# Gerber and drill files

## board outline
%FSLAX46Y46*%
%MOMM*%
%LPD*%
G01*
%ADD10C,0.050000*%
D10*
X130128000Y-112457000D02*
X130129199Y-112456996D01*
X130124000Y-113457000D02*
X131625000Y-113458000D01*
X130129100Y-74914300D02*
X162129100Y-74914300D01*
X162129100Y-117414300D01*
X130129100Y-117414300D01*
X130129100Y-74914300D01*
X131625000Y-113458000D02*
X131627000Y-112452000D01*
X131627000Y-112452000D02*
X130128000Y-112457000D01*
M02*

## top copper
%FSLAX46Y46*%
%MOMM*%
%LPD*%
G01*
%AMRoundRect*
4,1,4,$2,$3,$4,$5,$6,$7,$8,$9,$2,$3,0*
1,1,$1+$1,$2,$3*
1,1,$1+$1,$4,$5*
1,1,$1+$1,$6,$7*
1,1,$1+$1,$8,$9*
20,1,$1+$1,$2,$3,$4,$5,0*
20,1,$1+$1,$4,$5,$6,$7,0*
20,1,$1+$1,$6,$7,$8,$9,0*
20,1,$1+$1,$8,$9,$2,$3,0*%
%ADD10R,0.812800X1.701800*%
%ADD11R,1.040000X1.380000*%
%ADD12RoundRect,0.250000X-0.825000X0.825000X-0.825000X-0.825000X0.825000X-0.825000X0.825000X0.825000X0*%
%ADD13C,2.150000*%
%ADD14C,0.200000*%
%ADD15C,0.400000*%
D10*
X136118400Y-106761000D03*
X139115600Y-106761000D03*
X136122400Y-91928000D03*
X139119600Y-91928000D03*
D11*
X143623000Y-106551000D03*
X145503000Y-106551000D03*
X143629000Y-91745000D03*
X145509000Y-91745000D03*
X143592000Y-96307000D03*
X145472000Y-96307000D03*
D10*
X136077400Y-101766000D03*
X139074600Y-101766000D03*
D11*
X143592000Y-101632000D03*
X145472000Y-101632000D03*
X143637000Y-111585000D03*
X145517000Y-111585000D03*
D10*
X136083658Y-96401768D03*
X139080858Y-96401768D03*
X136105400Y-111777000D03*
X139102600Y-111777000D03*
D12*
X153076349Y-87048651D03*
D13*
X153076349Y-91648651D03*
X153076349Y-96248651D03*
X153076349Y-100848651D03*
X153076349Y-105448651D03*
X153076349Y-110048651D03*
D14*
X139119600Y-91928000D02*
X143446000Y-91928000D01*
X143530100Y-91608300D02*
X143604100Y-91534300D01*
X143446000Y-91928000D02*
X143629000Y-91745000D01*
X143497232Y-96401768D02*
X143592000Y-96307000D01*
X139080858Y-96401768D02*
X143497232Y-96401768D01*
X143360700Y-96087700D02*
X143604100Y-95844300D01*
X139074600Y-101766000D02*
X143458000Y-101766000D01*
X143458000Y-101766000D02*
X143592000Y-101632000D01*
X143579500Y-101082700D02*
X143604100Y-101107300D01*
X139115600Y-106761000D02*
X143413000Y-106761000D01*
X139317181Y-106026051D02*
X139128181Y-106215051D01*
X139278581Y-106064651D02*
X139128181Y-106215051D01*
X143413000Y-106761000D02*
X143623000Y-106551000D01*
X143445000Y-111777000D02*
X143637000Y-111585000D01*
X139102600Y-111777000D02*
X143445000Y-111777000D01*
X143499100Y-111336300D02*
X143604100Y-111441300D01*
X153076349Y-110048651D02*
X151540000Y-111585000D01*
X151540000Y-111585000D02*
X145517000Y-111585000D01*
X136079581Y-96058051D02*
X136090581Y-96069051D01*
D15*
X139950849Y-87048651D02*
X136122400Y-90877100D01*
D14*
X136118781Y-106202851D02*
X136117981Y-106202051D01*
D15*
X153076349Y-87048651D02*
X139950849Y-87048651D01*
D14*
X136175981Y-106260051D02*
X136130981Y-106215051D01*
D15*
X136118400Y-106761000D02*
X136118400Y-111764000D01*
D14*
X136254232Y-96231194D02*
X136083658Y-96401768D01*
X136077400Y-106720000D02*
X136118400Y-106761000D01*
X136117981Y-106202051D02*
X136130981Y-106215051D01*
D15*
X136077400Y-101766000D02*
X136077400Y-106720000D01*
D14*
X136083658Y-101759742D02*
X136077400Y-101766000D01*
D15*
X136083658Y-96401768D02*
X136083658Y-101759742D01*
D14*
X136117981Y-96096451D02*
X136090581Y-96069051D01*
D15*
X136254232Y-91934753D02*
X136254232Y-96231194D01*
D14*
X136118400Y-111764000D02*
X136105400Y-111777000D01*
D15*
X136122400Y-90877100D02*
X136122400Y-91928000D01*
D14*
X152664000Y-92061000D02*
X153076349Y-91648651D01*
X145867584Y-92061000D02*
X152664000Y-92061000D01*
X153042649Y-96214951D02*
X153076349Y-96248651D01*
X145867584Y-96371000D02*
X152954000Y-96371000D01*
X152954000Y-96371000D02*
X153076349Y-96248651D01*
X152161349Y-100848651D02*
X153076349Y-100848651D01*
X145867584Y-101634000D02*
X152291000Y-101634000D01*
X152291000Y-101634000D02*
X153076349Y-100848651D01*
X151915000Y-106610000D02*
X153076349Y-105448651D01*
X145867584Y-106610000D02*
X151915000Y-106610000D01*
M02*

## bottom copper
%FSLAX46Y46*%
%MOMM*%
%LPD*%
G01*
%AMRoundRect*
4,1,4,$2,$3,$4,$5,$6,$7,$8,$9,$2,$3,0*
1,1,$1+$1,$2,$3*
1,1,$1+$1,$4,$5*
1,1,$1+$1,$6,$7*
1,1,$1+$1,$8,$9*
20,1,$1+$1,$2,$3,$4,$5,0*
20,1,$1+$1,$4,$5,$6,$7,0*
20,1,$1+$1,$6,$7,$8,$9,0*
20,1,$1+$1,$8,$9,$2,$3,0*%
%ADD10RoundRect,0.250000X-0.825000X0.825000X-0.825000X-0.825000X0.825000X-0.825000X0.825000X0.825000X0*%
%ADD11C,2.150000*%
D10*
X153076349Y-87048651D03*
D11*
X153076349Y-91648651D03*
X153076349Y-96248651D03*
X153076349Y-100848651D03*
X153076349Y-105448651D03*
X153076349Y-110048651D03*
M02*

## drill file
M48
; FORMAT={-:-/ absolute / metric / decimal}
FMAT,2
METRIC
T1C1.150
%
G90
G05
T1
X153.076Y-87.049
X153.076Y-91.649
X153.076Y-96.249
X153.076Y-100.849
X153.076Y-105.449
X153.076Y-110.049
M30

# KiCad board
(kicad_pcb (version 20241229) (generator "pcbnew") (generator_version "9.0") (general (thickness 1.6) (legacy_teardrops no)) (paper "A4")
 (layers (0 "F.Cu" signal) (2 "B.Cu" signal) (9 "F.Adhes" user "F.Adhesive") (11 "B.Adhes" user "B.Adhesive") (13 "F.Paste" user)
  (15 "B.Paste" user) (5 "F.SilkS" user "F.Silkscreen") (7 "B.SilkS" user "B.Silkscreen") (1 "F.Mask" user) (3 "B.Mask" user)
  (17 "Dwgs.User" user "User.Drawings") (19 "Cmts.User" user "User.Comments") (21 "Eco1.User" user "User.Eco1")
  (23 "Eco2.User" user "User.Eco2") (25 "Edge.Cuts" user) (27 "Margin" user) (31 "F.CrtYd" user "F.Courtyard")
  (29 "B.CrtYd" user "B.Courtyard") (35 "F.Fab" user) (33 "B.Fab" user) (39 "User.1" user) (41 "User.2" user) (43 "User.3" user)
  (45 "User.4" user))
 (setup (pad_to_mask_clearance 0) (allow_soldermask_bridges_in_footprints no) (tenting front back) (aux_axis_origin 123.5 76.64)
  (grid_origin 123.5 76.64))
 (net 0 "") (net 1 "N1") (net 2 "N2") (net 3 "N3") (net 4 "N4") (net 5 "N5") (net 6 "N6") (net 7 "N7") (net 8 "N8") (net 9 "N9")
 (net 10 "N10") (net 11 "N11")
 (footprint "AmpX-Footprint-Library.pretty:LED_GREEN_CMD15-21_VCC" (layer "F.Cu") (at 137.617 106.761)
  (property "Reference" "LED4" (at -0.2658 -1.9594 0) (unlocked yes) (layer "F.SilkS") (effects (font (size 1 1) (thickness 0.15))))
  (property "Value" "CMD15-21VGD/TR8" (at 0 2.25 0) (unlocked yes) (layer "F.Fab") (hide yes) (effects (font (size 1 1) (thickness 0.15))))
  (pad "1" smd rect (at -1.4986 0) (size 0.8128 1.7018) (layers "F.Cu" "F.Mask" "F.Paste") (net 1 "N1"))
  (pad "2" smd rect (at 1.4986 0) (size 0.8128 1.7018) (layers "F.Cu" "F.Mask" "F.Paste") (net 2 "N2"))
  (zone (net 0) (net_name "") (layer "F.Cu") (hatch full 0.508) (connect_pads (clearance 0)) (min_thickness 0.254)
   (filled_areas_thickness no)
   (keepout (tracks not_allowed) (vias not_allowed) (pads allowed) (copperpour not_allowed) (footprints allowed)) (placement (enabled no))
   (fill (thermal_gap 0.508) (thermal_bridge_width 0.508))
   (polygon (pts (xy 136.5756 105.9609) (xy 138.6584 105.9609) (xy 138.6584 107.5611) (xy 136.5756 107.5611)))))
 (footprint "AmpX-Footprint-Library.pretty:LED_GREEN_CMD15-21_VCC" (layer "F.Cu") (at 137.621 91.928)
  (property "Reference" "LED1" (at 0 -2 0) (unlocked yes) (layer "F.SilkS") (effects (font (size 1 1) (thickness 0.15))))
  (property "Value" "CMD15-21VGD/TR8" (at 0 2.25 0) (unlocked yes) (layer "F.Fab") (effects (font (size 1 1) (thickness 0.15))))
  (pad "1" smd rect (at -1.4986 0) (size 0.8128 1.7018) (layers "F.Cu" "F.Mask" "F.Paste") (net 1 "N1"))
  (pad "2" smd rect (at 1.4986 0) (size 0.8128 1.7018) (layers "F.Cu" "F.Mask" "F.Paste") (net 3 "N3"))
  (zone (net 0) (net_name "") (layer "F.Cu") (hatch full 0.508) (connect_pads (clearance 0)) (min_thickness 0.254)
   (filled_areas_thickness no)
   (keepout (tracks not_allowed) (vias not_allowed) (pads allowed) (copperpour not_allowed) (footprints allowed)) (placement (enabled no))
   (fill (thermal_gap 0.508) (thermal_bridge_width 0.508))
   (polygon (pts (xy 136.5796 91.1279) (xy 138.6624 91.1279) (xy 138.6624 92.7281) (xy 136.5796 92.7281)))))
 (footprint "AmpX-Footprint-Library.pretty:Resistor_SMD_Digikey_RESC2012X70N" (layer "F.Cu") (at 144.563 106.551)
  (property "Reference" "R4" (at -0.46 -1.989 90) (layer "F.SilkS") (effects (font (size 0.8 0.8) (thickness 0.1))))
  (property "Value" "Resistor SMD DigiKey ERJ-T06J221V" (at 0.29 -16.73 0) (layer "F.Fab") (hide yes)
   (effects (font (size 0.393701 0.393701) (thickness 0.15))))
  (pad "1" smd rect (at -0.94 0) (size 1.04 1.38) (layers "F.Cu" "F.Mask" "F.Paste") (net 2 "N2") (solder_mask_margin 0.102))
  (pad "2" smd rect (at 0.94 0) (size 1.04 1.38) (layers "F.Cu" "F.Mask" "F.Paste") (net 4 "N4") (solder_mask_margin 0.102)))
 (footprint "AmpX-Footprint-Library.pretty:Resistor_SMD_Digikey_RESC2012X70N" (layer "F.Cu") (at 144.569 91.745)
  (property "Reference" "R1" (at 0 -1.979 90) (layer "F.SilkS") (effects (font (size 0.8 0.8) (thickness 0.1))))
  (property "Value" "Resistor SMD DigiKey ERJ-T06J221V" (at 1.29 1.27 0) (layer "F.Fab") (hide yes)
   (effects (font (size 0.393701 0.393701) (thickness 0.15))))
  (pad "1" smd rect (at -0.94 0) (size 1.04 1.38) (layers "F.Cu" "F.Mask" "F.Paste") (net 3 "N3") (solder_mask_margin 0.102))
  (pad "2" smd rect (at 0.94 0) (size 1.04 1.38) (layers "F.Cu" "F.Mask" "F.Paste") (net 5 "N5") (solder_mask_margin 0.102)))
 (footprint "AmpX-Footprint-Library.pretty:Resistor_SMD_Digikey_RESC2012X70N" (layer "F.Cu") (at 144.532 96.307)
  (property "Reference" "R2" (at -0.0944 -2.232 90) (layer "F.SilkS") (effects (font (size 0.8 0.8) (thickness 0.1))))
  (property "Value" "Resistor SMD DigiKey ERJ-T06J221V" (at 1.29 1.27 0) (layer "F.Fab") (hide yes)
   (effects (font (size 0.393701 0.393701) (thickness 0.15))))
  (pad "1" smd rect (at -0.94 0) (size 1.04 1.38) (layers "F.Cu" "F.Mask" "F.Paste") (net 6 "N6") (solder_mask_margin 0.102))
  (pad "2" smd rect (at 0.94 0) (size 1.04 1.38) (layers "F.Cu" "F.Mask" "F.Paste") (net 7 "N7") (solder_mask_margin 0.102)))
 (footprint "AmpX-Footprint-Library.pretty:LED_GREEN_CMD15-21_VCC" (layer "F.Cu") (at 137.576 101.766)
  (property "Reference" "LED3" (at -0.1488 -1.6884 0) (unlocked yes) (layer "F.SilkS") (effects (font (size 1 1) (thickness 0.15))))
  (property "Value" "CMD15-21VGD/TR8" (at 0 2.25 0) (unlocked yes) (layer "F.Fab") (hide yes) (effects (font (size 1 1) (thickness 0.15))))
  (pad "1" smd rect (at -1.4986 0) (size 0.8128 1.7018) (layers "F.Cu" "F.Mask" "F.Paste") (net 1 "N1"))
  (pad "2" smd rect (at 1.4986 0) (size 0.8128 1.7018) (layers "F.Cu" "F.Mask" "F.Paste") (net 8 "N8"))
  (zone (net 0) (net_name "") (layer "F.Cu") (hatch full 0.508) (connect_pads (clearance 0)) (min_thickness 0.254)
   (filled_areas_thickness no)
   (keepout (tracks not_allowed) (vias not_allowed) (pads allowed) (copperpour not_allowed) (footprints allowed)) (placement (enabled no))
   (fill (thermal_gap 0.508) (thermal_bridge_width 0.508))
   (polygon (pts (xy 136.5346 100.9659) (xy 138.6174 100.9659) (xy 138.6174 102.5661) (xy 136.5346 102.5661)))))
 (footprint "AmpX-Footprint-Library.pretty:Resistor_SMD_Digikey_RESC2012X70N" (layer "F.Cu") (at 144.532 101.632)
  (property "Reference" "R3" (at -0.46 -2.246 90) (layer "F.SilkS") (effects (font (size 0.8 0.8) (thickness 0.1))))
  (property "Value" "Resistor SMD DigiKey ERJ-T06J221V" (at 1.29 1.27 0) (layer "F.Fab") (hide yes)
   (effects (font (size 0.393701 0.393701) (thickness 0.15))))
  (pad "1" smd rect (at -0.94 0) (size 1.04 1.38) (layers "F.Cu" "F.Mask" "F.Paste") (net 8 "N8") (solder_mask_margin 0.102))
  (pad "2" smd rect (at 0.94 0) (size 1.04 1.38) (layers "F.Cu" "F.Mask" "F.Paste") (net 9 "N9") (solder_mask_margin 0.102)))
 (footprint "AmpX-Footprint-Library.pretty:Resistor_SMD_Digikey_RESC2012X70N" (layer "F.Cu") (at 144.577 111.585)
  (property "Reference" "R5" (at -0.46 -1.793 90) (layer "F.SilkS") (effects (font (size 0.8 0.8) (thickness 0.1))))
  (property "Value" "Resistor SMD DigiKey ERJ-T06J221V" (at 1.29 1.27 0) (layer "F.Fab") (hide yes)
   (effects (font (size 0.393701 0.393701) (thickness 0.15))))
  (pad "1" smd rect (at -0.94 0) (size 1.04 1.38) (layers "F.Cu" "F.Mask" "F.Paste") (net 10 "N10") (solder_mask_margin 0.102))
  (pad "2" smd rect (at 0.94 0) (size 1.04 1.38) (layers "F.Cu" "F.Mask" "F.Paste") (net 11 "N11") (solder_mask_margin 0.102)))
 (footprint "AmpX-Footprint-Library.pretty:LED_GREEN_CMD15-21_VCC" (layer "F.Cu") (at 137.582258 96.401768)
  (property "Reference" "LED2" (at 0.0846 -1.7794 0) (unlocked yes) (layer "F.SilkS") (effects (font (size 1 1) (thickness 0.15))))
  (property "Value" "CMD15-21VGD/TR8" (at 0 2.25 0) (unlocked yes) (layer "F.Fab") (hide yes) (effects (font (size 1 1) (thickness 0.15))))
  (pad "1" smd rect (at -1.4986 0) (size 0.8128 1.7018) (layers "F.Cu" "F.Mask" "F.Paste") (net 1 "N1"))
  (pad "2" smd rect (at 1.4986 0) (size 0.8128 1.7018) (layers "F.Cu" "F.Mask" "F.Paste") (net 6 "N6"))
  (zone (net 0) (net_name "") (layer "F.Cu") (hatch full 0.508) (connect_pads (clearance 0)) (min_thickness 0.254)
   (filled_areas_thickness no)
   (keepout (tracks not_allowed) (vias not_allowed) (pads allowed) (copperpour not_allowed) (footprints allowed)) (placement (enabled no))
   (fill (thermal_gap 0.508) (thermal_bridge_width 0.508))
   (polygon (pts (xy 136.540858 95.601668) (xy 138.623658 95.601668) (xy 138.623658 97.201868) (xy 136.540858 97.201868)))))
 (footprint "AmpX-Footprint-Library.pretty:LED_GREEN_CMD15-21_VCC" (layer "F.Cu") (at 137.604 111.777)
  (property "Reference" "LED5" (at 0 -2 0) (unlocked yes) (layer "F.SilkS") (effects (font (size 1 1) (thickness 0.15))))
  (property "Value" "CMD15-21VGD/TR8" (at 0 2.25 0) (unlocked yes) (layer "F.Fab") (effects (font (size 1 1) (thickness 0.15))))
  (pad "1" smd rect (at -1.4986 0) (size 0.8128 1.7018) (layers "F.Cu" "F.Mask" "F.Paste") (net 1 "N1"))
  (pad "2" smd rect (at 1.4986 0) (size 0.8128 1.7018) (layers "F.Cu" "F.Mask" "F.Paste") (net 10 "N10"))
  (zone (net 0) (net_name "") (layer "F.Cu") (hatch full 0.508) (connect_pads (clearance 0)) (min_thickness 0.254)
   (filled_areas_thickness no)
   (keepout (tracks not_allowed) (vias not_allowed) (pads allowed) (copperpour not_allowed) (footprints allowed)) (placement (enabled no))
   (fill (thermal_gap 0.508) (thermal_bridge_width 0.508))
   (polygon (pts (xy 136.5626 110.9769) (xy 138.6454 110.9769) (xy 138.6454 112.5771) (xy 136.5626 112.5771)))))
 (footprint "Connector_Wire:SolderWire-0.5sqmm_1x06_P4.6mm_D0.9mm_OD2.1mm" (layer "F.Cu") (at 153.076349 87.048651 -90)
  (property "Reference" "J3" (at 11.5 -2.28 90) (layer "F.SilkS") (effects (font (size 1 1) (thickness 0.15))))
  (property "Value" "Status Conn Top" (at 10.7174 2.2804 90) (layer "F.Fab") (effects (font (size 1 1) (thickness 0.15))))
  (pad "1" thru_hole roundrect (at 0 0 270) (size 2.15 2.15) (drill 1.15) (layers "*.Cu" "*.Mask") (remove_unused_layers no)
   (roundrect_rratio 0.116279) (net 1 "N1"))
  (pad "2" thru_hole circle (at 4.6 0 270) (size 2.15 2.15) (drill 1.15) (layers "*.Cu" "*.Mask") (remove_unused_layers no) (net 5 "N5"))
  (pad "3" thru_hole circle (at 9.2 0 270) (size 2.15 2.15) (drill 1.15) (layers "*.Cu" "*.Mask") (remove_unused_layers no) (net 7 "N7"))
  (pad "4" thru_hole circle (at 13.8 0 270) (size 2.15 2.15) (drill 1.15) (layers "*.Cu" "*.Mask") (remove_unused_layers no) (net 9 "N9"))
  (pad "5" thru_hole circle (at 18.4 0 270) (size 2.15 2.15) (drill 1.15) (layers "*.Cu" "*.Mask") (remove_unused_layers no) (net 4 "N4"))
  (pad "6" thru_hole circle (at 23 0 270) (size 2.15 2.15) (drill 1.15) (layers "*.Cu" "*.Mask") (remove_unused_layers no) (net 11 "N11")))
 (gr_line (start 130.128 112.457) (end 130.129199 112.456996) (stroke (width 0.05) (type default)) (layer "Edge.Cuts"))
 (gr_line (start 130.124 113.457) (end 131.625 113.458) (stroke (width 0.05) (type default)) (layer "Edge.Cuts"))
 (gr_rect (start 130.1291 74.9143) (end 162.1291 117.4143) (stroke (width 0.05) (type default)) (fill no) (layer "Edge.Cuts"))
 (gr_line (start 131.625 113.458) (end 131.627 112.452) (stroke (width 0.05) (type default)) (layer "Edge.Cuts"))
 (gr_line (start 131.627 112.452) (end 130.128 112.457) (stroke (width 0.05) (type default)) (layer "Edge.Cuts"))
 (segment (start 139.1196 91.928) (end 143.446 91.928) (width 0.2) (layer "F.Cu") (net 3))
 (segment (start 143.5301 91.6083) (end 143.6041 91.5343) (width 0.2) (layer "F.Cu") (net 3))
 (segment (start 143.446 91.928) (end 143.629 91.745) (width 0.2) (layer "F.Cu") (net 3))
 (segment (start 143.497232 96.401768) (end 143.592 96.307) (width 0.2) (layer "F.Cu") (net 6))
 (segment (start 139.080858 96.401768) (end 143.497232 96.401768) (width 0.2) (layer "F.Cu") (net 6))
 (segment (start 143.3607 96.0877) (end 143.6041 95.8443) (width 0.2) (layer "F.Cu") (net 6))
 (segment (start 139.0746 101.766) (end 143.458 101.766) (width 0.2) (layer "F.Cu") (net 8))
 (segment (start 143.458 101.766) (end 143.592 101.632) (width 0.2) (layer "F.Cu") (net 8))
 (segment (start 143.5795 101.0827) (end 143.6041 101.1073) (width 0.2) (layer "F.Cu") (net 8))
 (segment (start 139.1156 106.761) (end 143.413 106.761) (width 0.2) (layer "F.Cu") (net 2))
 (segment (start 139.317181 106.026051) (end 139.128181 106.215051) (width 0.2) (layer "F.Cu") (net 2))
 (segment (start 139.278581 106.064651) (end 139.128181 106.215051) (width 0.2) (layer "F.Cu") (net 2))
 (segment (start 143.413 106.761) (end 143.623 106.551) (width 0.2) (layer "F.Cu") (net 2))
 (segment (start 143.445 111.777) (end 143.637 111.585) (width 0.2) (layer "F.Cu") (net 10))
 (segment (start 139.1026 111.777) (end 143.445 111.777) (width 0.2) (layer "F.Cu") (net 10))
 (segment (start 143.4991 111.3363) (end 143.6041 111.4413) (width 0.2) (layer "F.Cu") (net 10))
 (segment (start 153.076349 110.048651) (end 151.54 111.585) (width 0.2) (layer "F.Cu") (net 11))
 (segment (start 151.54 111.585) (end 145.517 111.585) (width 0.2) (layer "F.Cu") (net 11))
 (segment (start 136.079581 96.058051) (end 136.090581 96.069051) (width 0.2) (layer "F.Cu") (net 1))
 (segment (start 139.950849 87.048651) (end 136.1224 90.8771) (width 0.4) (layer "F.Cu") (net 1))
 (segment (start 136.118781 106.202851) (end 136.117981 106.202051) (width 0.2) (layer "F.Cu") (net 1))
 (segment (start 153.076349 87.048651) (end 139.950849 87.048651) (width 0.4) (layer "F.Cu") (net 1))
 (segment (start 136.175981 106.260051) (end 136.130981 106.215051) (width 0.2) (layer "F.Cu") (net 1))
 (segment (start 136.1184 106.761) (end 136.1184 111.764) (width 0.4) (layer "F.Cu") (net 1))
 (segment (start 136.254232 96.231194) (end 136.083658 96.401768) (width 0.2) (layer "F.Cu") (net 1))
 (segment (start 136.0774 106.72) (end 136.1184 106.761) (width 0.2) (layer "F.Cu") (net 1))
 (segment (start 136.117981 106.202051) (end 136.130981 106.215051) (width 0.2) (layer "F.Cu") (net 1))
 (segment (start 136.0774 101.766) (end 136.0774 106.72) (width 0.4) (layer "F.Cu") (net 1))
 (segment (start 136.083658 101.759742) (end 136.0774 101.766) (width 0.2) (layer "F.Cu") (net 1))
 (segment (start 136.083658 96.401768) (end 136.083658 101.759742) (width 0.4) (layer "F.Cu") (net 1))
 (segment (start 136.117981 96.096451) (end 136.090581 96.069051) (width 0.2) (layer "F.Cu") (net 1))
 (segment (start 136.254232 91.934753) (end 136.254232 96.231194) (width 0.4) (layer "F.Cu") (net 1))
 (segment (start 136.1184 111.764) (end 136.1054 111.777) (width 0.2) (layer "F.Cu") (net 1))
 (segment (start 136.1224 90.8771) (end 136.1224 91.928) (width 0.4) (layer "F.Cu") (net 1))
 (segment (start 152.664 92.061) (end 153.076349 91.648651) (width 0.2) (layer "F.Cu") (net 5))
 (segment (start 145.867584 92.061) (end 152.664 92.061) (width 0.2) (layer "F.Cu") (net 5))
 (segment (start 153.042649 96.214951) (end 153.076349 96.248651) (width 0.2) (layer "F.Cu") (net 7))
 (segment (start 145.867584 96.371) (end 152.954 96.371) (width 0.2) (layer "F.Cu") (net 7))
 (segment (start 152.954 96.371) (end 153.076349 96.248651) (width 0.2) (layer "F.Cu") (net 7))
 (segment (start 152.161349 100.848651) (end 153.076349 100.848651) (width 0.2) (layer "F.Cu") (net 9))
 (segment (start 145.867584 101.634) (end 152.291 101.634) (width 0.2) (layer "F.Cu") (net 9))
 (segment (start 152.291 101.634) (end 153.076349 100.848651) (width 0.2) (layer "F.Cu") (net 9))
 (segment (start 151.915 106.61) (end 153.076349 105.448651) (width 0.2) (layer "F.Cu") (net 4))
 (segment (start 145.867584 106.61) (end 151.915 106.61) (width 0.2) (layer "F.Cu") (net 4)))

